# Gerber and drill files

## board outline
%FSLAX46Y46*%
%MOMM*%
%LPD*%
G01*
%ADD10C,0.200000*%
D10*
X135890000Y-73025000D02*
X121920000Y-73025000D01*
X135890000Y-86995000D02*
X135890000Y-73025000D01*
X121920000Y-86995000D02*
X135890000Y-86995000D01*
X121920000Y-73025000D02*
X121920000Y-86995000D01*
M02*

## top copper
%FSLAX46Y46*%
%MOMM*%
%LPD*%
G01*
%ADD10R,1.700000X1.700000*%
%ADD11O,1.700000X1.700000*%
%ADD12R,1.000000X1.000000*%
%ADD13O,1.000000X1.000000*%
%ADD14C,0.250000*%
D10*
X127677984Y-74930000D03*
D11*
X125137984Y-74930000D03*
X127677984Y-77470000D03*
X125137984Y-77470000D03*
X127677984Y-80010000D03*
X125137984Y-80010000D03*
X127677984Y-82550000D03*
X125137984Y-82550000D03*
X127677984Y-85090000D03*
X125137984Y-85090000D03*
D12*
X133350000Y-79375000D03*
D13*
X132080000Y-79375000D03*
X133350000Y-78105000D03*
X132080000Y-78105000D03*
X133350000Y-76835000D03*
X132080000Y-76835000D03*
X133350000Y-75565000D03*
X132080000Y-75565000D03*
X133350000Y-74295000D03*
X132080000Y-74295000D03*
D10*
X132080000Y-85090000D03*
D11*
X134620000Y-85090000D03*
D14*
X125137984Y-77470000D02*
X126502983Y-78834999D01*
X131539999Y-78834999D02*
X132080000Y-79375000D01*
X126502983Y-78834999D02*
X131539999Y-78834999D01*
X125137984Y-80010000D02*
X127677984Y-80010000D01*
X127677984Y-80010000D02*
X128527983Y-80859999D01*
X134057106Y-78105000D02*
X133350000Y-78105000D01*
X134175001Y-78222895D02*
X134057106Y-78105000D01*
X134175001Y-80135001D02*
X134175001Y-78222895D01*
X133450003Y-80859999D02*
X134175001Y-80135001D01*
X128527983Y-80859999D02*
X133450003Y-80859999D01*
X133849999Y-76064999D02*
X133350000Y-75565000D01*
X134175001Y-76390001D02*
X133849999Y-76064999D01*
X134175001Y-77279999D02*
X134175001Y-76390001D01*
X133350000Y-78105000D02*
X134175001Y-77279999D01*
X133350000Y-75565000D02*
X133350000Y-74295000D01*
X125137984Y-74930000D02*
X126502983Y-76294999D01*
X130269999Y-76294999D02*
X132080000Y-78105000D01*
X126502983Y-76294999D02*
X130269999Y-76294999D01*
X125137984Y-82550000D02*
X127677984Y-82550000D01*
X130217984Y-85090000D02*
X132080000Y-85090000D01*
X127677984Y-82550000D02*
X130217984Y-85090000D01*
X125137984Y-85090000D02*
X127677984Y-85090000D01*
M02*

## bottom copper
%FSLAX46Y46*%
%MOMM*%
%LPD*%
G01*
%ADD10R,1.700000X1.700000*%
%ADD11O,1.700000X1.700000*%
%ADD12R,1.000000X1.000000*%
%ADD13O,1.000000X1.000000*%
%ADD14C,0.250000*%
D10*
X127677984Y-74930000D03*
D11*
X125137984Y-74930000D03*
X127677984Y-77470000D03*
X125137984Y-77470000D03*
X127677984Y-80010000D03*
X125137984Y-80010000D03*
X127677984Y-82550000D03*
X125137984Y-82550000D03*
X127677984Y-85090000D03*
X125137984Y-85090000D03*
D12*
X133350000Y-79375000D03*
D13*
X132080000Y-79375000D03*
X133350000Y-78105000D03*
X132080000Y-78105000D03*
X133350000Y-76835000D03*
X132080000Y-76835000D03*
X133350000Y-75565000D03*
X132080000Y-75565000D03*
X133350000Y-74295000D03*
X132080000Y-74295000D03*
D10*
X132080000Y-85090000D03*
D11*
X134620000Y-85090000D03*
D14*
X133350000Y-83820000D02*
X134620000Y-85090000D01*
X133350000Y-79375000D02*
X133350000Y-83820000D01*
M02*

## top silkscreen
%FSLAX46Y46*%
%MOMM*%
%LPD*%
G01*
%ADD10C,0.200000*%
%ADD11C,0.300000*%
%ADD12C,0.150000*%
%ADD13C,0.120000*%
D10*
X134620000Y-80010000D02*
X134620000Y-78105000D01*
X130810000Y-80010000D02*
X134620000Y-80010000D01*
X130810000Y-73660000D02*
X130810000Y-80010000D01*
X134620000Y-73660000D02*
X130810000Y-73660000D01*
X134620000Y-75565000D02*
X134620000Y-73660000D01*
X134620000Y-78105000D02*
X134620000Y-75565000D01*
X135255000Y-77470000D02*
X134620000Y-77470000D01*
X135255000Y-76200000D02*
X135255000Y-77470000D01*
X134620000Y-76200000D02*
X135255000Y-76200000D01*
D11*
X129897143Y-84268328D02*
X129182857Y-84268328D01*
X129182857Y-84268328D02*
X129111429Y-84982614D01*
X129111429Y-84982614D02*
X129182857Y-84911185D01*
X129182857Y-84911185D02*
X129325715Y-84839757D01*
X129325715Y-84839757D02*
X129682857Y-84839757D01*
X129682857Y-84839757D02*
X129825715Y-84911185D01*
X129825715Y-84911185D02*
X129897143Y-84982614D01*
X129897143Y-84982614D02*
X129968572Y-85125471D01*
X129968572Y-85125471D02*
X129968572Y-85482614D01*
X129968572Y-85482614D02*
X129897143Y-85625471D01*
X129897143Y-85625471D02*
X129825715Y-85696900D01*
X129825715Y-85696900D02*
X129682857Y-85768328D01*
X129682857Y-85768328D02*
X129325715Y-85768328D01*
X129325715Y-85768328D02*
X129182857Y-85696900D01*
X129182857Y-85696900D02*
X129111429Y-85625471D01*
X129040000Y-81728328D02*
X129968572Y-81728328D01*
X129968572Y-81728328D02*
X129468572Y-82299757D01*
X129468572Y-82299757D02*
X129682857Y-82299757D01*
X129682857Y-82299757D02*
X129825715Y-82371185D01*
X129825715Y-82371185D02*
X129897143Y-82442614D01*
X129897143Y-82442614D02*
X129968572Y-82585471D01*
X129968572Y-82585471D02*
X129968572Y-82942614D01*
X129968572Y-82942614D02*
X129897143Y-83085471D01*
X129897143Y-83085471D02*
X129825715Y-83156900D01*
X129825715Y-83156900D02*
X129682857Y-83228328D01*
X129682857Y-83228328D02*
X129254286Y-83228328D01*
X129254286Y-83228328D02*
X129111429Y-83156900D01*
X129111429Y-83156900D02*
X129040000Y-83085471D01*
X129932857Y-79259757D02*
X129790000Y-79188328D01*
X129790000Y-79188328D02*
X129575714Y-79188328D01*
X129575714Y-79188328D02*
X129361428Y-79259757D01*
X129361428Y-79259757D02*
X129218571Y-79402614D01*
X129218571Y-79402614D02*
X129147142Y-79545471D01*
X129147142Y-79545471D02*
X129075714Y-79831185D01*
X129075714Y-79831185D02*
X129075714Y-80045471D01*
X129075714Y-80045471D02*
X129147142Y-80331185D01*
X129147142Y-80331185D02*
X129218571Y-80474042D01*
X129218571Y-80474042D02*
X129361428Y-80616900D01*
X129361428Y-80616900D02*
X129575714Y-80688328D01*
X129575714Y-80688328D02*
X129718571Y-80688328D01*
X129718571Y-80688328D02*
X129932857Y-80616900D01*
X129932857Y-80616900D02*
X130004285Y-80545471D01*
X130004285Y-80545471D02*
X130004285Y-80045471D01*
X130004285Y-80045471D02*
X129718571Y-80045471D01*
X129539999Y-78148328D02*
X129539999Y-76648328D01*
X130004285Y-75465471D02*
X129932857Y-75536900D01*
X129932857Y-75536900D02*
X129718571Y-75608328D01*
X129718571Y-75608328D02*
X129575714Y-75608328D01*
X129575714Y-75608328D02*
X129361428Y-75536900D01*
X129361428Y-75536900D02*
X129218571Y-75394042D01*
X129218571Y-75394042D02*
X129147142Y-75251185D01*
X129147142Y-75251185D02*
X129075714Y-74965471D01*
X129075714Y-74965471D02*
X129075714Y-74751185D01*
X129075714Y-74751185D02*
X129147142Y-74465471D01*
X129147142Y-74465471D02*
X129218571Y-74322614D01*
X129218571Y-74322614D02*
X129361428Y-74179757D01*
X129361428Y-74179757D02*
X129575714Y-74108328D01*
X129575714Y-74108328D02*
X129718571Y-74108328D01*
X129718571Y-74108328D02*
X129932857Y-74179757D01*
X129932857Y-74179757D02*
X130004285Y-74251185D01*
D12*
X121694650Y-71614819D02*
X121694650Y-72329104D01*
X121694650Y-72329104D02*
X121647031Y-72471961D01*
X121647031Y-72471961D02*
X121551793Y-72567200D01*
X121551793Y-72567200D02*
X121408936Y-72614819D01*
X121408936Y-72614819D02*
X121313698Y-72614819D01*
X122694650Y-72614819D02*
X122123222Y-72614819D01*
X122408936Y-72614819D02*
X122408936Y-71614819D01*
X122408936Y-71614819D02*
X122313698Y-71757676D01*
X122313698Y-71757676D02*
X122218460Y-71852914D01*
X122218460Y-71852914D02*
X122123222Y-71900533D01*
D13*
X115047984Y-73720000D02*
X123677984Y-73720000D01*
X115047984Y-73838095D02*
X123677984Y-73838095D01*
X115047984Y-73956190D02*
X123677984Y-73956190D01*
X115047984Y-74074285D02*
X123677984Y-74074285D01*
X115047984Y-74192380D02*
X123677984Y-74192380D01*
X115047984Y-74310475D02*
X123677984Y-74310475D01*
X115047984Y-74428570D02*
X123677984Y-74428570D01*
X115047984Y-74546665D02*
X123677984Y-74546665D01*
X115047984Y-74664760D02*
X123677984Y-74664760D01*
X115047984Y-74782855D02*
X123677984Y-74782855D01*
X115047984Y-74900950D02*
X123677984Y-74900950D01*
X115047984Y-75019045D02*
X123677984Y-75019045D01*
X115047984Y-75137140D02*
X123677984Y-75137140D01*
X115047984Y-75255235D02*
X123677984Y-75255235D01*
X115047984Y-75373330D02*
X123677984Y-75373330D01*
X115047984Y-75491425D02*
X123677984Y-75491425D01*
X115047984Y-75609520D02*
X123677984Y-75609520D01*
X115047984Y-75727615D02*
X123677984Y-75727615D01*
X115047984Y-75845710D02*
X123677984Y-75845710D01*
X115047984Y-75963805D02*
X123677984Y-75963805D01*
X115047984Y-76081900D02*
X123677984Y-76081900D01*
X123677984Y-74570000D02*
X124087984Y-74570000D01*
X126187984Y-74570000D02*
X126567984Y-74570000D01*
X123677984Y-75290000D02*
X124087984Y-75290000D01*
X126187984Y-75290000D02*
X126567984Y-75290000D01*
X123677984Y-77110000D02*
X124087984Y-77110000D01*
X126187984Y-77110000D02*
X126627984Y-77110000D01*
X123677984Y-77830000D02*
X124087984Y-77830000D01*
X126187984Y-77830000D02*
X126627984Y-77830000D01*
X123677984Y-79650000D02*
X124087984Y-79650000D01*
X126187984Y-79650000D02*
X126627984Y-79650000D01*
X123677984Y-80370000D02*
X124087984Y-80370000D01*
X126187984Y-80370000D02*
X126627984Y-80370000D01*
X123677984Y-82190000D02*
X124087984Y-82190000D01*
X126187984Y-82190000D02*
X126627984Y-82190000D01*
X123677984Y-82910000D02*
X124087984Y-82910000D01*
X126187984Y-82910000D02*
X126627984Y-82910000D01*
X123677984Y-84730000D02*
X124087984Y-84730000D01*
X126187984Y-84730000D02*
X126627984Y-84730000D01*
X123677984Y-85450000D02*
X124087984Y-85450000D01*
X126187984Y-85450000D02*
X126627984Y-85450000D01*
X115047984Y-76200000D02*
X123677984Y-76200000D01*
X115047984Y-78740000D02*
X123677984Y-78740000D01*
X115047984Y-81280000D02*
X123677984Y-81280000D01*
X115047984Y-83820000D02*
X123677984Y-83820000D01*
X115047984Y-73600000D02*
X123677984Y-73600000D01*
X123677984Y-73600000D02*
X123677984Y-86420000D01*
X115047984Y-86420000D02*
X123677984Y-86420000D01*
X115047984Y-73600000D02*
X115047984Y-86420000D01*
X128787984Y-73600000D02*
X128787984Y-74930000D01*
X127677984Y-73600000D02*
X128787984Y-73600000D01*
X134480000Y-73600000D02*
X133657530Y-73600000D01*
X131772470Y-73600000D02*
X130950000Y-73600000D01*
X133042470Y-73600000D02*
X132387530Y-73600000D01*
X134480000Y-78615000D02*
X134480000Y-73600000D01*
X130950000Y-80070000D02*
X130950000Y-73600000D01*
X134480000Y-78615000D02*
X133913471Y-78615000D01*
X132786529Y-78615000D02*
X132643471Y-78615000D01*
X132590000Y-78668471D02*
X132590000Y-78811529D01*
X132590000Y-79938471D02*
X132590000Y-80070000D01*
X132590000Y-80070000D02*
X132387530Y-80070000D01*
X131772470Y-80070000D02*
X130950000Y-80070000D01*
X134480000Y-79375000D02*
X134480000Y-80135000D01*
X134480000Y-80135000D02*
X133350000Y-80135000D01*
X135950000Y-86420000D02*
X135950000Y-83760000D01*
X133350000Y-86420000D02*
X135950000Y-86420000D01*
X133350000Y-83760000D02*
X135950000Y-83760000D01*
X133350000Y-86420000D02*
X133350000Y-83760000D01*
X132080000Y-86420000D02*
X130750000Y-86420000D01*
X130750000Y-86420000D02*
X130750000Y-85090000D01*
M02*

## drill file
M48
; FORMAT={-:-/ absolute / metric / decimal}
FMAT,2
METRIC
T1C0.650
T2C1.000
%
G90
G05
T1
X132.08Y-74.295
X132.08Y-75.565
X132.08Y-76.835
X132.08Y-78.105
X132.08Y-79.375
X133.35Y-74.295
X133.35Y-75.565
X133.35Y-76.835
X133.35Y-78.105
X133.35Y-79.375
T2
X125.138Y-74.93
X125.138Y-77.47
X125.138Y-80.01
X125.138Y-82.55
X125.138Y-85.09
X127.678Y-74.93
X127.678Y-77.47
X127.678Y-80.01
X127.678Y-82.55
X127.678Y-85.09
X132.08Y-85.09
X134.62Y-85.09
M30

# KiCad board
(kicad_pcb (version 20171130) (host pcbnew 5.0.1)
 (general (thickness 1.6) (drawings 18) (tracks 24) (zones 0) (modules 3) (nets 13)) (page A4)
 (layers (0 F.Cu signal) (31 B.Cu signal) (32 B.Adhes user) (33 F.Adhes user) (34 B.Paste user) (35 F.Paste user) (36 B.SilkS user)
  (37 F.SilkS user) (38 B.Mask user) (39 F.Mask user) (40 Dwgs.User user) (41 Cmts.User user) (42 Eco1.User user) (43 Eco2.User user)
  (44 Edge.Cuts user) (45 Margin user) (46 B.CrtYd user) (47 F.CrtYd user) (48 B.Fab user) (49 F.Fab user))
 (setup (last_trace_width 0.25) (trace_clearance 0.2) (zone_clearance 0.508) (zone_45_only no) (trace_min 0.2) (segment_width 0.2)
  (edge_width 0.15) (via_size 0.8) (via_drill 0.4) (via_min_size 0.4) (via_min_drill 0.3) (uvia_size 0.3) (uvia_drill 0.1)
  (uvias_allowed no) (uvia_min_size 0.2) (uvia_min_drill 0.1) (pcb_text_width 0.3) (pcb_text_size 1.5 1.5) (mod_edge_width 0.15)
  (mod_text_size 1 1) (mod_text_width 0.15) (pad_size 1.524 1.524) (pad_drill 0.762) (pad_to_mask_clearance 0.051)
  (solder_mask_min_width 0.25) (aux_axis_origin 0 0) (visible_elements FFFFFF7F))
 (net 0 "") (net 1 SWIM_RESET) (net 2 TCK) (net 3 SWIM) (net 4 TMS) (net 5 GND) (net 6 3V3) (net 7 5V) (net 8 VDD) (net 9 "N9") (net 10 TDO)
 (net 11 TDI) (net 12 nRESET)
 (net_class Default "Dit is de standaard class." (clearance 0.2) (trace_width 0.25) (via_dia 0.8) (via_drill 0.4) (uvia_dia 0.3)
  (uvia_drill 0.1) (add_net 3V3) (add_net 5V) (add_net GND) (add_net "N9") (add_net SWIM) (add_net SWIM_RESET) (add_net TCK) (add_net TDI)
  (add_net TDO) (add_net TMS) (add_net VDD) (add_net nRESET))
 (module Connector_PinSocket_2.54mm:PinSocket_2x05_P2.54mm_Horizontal (layer F.Cu) (at 127.677984 74.93)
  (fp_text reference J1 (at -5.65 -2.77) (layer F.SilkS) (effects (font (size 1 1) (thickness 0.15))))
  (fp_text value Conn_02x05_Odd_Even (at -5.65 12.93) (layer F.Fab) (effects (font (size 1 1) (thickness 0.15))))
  (fp_line (start -12.63 -1.21) (end -4 -1.21) (layer F.SilkS) (width 0.12))
  (fp_line (start -12.63 -1.091905) (end -4 -1.091905) (layer F.SilkS) (width 0.12))
  (fp_line (start -12.63 -0.97381) (end -4 -0.97381) (layer F.SilkS) (width 0.12))
  (fp_line (start -12.63 -0.855715) (end -4 -0.855715) (layer F.SilkS) (width 0.12))
  (fp_line (start -12.63 -0.73762) (end -4 -0.73762) (layer F.SilkS) (width 0.12))
  (fp_line (start -12.63 -0.619525) (end -4 -0.619525) (layer F.SilkS) (width 0.12))
  (fp_line (start -12.63 -0.50143) (end -4 -0.50143) (layer F.SilkS) (width 0.12))
  (fp_line (start -12.63 -0.383335) (end -4 -0.383335) (layer F.SilkS) (width 0.12))
  (fp_line (start -12.63 -0.26524) (end -4 -0.26524) (layer F.SilkS) (width 0.12))
  (fp_line (start -12.63 -0.147145) (end -4 -0.147145) (layer F.SilkS) (width 0.12))
  (fp_line (start -12.63 -0.02905) (end -4 -0.02905) (layer F.SilkS) (width 0.12))
  (fp_line (start -12.63 0.089045) (end -4 0.089045) (layer F.SilkS) (width 0.12))
  (fp_line (start -12.63 0.20714) (end -4 0.20714) (layer F.SilkS) (width 0.12))
  (fp_line (start -12.63 0.325235) (end -4 0.325235) (layer F.SilkS) (width 0.12))
  (fp_line (start -12.63 0.44333) (end -4 0.44333) (layer F.SilkS) (width 0.12))
  (fp_line (start -12.63 0.561425) (end -4 0.561425) (layer F.SilkS) (width 0.12))
  (fp_line (start -12.63 0.67952) (end -4 0.67952) (layer F.SilkS) (width 0.12))
  (fp_line (start -12.63 0.797615) (end -4 0.797615) (layer F.SilkS) (width 0.12))
  (fp_line (start -12.63 0.91571) (end -4 0.91571) (layer F.SilkS) (width 0.12))
  (fp_line (start -12.63 1.033805) (end -4 1.033805) (layer F.SilkS) (width 0.12))
  (fp_line (start -12.63 1.1519) (end -4 1.1519) (layer F.SilkS) (width 0.12))
  (fp_line (start -4 -0.36) (end -3.59 -0.36) (layer F.SilkS) (width 0.12))
  (fp_line (start -1.49 -0.36) (end -1.11 -0.36) (layer F.SilkS) (width 0.12))
  (fp_line (start -4 0.36) (end -3.59 0.36) (layer F.SilkS) (width 0.12))
  (fp_line (start -1.49 0.36) (end -1.11 0.36) (layer F.SilkS) (width 0.12))
  (fp_line (start -4 2.18) (end -3.59 2.18) (layer F.SilkS) (width 0.12))
  (fp_line (start -1.49 2.18) (end -1.05 2.18) (layer F.SilkS) (width 0.12))
  (fp_line (start -4 2.9) (end -3.59 2.9) (layer F.SilkS) (width 0.12))
  (fp_line (start -1.49 2.9) (end -1.05 2.9) (layer F.SilkS) (width 0.12))
  (fp_line (start -4 4.72) (end -3.59 4.72) (layer F.SilkS) (width 0.12))
  (fp_line (start -1.49 4.72) (end -1.05 4.72) (layer F.SilkS) (width 0.12))
  (fp_line (start -4 5.44) (end -3.59 5.44) (layer F.SilkS) (width 0.12))
  (fp_line (start -1.49 5.44) (end -1.05 5.44) (layer F.SilkS) (width 0.12))
  (fp_line (start -4 7.26) (end -3.59 7.26) (layer F.SilkS) (width 0.12))
  (fp_line (start -1.49 7.26) (end -1.05 7.26) (layer F.SilkS) (width 0.12))
  (fp_line (start -4 7.98) (end -3.59 7.98) (layer F.SilkS) (width 0.12))
  (fp_line (start -1.49 7.98) (end -1.05 7.98) (layer F.SilkS) (width 0.12))
  (fp_line (start -4 9.8) (end -3.59 9.8) (layer F.SilkS) (width 0.12))
  (fp_line (start -1.49 9.8) (end -1.05 9.8) (layer F.SilkS) (width 0.12))
  (fp_line (start -4 10.52) (end -3.59 10.52) (layer F.SilkS) (width 0.12))
  (fp_line (start -1.49 10.52) (end -1.05 10.52) (layer F.SilkS) (width 0.12))
  (fp_line (start -12.63 1.27) (end -4 1.27) (layer F.SilkS) (width 0.12))
  (fp_line (start -12.63 3.81) (end -4 3.81) (layer F.SilkS) (width 0.12))
  (fp_line (start -12.63 6.35) (end -4 6.35) (layer F.SilkS) (width 0.12))
  (fp_line (start -12.63 8.89) (end -4 8.89) (layer F.SilkS) (width 0.12))
  (fp_line (start -12.63 -1.33) (end -4 -1.33) (layer F.SilkS) (width 0.12))
  (fp_line (start -4 -1.33) (end -4 11.49) (layer F.SilkS) (width 0.12))
  (fp_line (start -12.63 11.49) (end -4 11.49) (layer F.SilkS) (width 0.12))
  (fp_line (start -12.63 -1.33) (end -12.63 11.49) (layer F.SilkS) (width 0.12))
  (fp_line (start 1.11 -1.33) (end 1.11 0) (layer F.SilkS) (width 0.12))
  (fp_line (start 0 -1.33) (end 1.11 -1.33) (layer F.SilkS) (width 0.12))
  (pad 1 thru_hole rect (at 0 0) (size 1.7 1.7) (drill 1) (layers *.Cu *.Mask) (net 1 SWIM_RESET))
  (pad 2 thru_hole oval (at -2.54 0) (size 1.7 1.7) (drill 1) (layers *.Cu *.Mask) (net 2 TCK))
  (pad 3 thru_hole oval (at 0 2.54) (size 1.7 1.7) (drill 1) (layers *.Cu *.Mask) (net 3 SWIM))
  (pad 4 thru_hole oval (at -2.54 2.54) (size 1.7 1.7) (drill 1) (layers *.Cu *.Mask) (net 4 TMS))
  (pad 5 thru_hole oval (at 0 5.08) (size 1.7 1.7) (drill 1) (layers *.Cu *.Mask) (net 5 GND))
  (pad 6 thru_hole oval (at -2.54 5.08) (size 1.7 1.7) (drill 1) (layers *.Cu *.Mask) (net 5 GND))
  (pad 7 thru_hole oval (at 0 7.62) (size 1.7 1.7) (drill 1) (layers *.Cu *.Mask) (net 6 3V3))
  (pad 8 thru_hole oval (at -2.54 7.62) (size 1.7 1.7) (drill 1) (layers *.Cu *.Mask) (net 6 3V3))
  (pad 9 thru_hole oval (at 0 10.16) (size 1.7 1.7) (drill 1) (layers *.Cu *.Mask) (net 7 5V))
  (pad 10 thru_hole oval (at -2.54 10.16) (size 1.7 1.7) (drill 1) (layers *.Cu *.Mask) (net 7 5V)))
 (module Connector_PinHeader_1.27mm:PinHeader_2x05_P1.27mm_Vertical (layer F.Cu) (at 133.35 79.375 180)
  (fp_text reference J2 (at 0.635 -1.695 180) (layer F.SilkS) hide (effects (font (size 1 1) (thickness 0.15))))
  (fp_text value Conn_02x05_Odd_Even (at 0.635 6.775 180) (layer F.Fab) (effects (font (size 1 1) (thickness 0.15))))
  (fp_line (start -1.13 5.775) (end -0.30753 5.775) (layer F.SilkS) (width 0.12))
  (fp_line (start 1.57753 5.775) (end 2.4 5.775) (layer F.SilkS) (width 0.12))
  (fp_line (start 0.30753 5.775) (end 0.96247 5.775) (layer F.SilkS) (width 0.12))
  (fp_line (start -1.13 0.76) (end -1.13 5.775) (layer F.SilkS) (width 0.12))
  (fp_line (start 2.4 -0.695) (end 2.4 5.775) (layer F.SilkS) (width 0.12))
  (fp_line (start -1.13 0.76) (end -0.563471 0.76) (layer F.SilkS) (width 0.12))
  (fp_line (start 0.563471 0.76) (end 0.706529 0.76) (layer F.SilkS) (width 0.12))
  (fp_line (start 0.76 0.706529) (end 0.76 0.563471) (layer F.SilkS) (width 0.12))
  (fp_line (start 0.76 -0.563471) (end 0.76 -0.695) (layer F.SilkS) (width 0.12))
  (fp_line (start 0.76 -0.695) (end 0.96247 -0.695) (layer F.SilkS) (width 0.12))
  (fp_line (start 1.57753 -0.695) (end 2.4 -0.695) (layer F.SilkS) (width 0.12))
  (fp_line (start -1.13 0) (end -1.13 -0.76) (layer F.SilkS) (width 0.12))
  (fp_line (start -1.13 -0.76) (end 0 -0.76) (layer F.SilkS) (width 0.12))
  (pad 1 thru_hole rect (at 0 0 180) (size 1 1) (drill 0.65) (layers *.Cu *.Mask) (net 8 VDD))
  (pad 2 thru_hole oval (at 1.27 0 180) (size 1 1) (drill 0.65) (layers *.Cu *.Mask) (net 4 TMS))
  (pad 3 thru_hole oval (at 0 1.27 180) (size 1 1) (drill 0.65) (layers *.Cu *.Mask) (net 5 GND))
  (pad 4 thru_hole oval (at 1.27 1.27 180) (size 1 1) (drill 0.65) (layers *.Cu *.Mask) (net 2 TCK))
  (pad 5 thru_hole oval (at 0 2.54 180) (size 1 1) (drill 0.65) (layers *.Cu *.Mask) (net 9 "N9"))
  (pad 6 thru_hole oval (at 1.27 2.54 180) (size 1 1) (drill 0.65) (layers *.Cu *.Mask) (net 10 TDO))
  (pad 7 thru_hole oval (at 0 3.81 180) (size 1 1) (drill 0.65) (layers *.Cu *.Mask) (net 5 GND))
  (pad 8 thru_hole oval (at 1.27 3.81 180) (size 1 1) (drill 0.65) (layers *.Cu *.Mask) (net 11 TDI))
  (pad 9 thru_hole oval (at 0 5.08 180) (size 1 1) (drill 0.65) (layers *.Cu *.Mask) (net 5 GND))
  (pad 10 thru_hole oval (at 1.27 5.08 180) (size 1 1) (drill 0.65) (layers *.Cu *.Mask) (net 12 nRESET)))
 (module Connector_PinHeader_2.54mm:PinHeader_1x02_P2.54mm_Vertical (layer F.Cu) (at 132.08 85.09 90)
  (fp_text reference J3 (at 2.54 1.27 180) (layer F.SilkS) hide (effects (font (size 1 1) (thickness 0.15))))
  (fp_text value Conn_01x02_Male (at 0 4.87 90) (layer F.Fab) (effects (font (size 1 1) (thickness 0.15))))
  (fp_line (start -1.33 3.87) (end 1.33 3.87) (layer F.SilkS) (width 0.12))
  (fp_line (start -1.33 1.27) (end -1.33 3.87) (layer F.SilkS) (width 0.12))
  (fp_line (start 1.33 1.27) (end 1.33 3.87) (layer F.SilkS) (width 0.12))
  (fp_line (start -1.33 1.27) (end 1.33 1.27) (layer F.SilkS) (width 0.12))
  (fp_line (start -1.33 0) (end -1.33 -1.33) (layer F.SilkS) (width 0.12))
  (fp_line (start -1.33 -1.33) (end 0 -1.33) (layer F.SilkS) (width 0.12))
  (pad 1 thru_hole rect (at 0 0 90) (size 1.7 1.7) (drill 1) (layers *.Cu *.Mask) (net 6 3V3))
  (pad 2 thru_hole oval (at 0 2.54 90) (size 1.7 1.7) (drill 1) (layers *.Cu *.Mask) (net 8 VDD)))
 (gr_line (start 134.62 80.01) (end 134.62 78.105) (layer F.SilkS) (width 0.2))
 (gr_line (start 130.81 80.01) (end 134.62 80.01) (layer F.SilkS) (width 0.2))
 (gr_line (start 130.81 73.66) (end 130.81 80.01) (layer F.SilkS) (width 0.2))
 (gr_line (start 134.62 73.66) (end 130.81 73.66) (layer F.SilkS) (width 0.2))
 (gr_line (start 134.62 75.565) (end 134.62 73.66) (layer F.SilkS) (width 0.2))
 (gr_line (start 134.62 78.105) (end 134.62 75.565) (layer F.SilkS) (width 0.2))
 (gr_line (start 135.255 77.47) (end 134.62 77.47) (layer F.SilkS) (width 0.2))
 (gr_line (start 135.255 76.2) (end 135.255 77.47) (layer F.SilkS) (width 0.2))
 (gr_line (start 134.62 76.2) (end 135.255 76.2) (layer F.SilkS) (width 0.2))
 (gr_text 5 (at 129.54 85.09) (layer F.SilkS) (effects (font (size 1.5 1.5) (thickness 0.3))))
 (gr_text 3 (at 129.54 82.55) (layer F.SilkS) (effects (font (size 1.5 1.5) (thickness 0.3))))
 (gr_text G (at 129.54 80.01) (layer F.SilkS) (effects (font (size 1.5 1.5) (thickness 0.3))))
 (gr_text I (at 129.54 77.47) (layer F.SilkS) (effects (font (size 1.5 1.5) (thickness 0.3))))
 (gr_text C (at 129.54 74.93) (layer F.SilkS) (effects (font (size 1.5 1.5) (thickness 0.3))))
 (gr_line (start 135.89 73.025) (end 121.92 73.025) (layer Edge.Cuts) (width 0.2))
 (gr_line (start 135.89 86.995) (end 135.89 73.025) (layer Edge.Cuts) (width 0.2))
 (gr_line (start 121.92 86.995) (end 135.89 86.995) (layer Edge.Cuts) (width 0.2))
 (gr_line (start 121.92 73.025) (end 121.92 86.995) (layer Edge.Cuts) (width 0.2))
 (segment (start 125.137984 77.47) (end 126.502983 78.834999) (width 0.25) (layer F.Cu) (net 4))
 (segment (start 131.539999 78.834999) (end 132.08 79.375) (width 0.25) (layer F.Cu) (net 4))
 (segment (start 126.502983 78.834999) (end 131.539999 78.834999) (width 0.25) (layer F.Cu) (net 4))
 (segment (start 125.137984 80.01) (end 127.677984 80.01) (width 0.25) (layer F.Cu) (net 5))
 (segment (start 127.677984 80.01) (end 128.527983 80.859999) (width 0.25) (layer F.Cu) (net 5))
 (segment (start 134.057106 78.105) (end 133.35 78.105) (width 0.25) (layer F.Cu) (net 5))
 (segment (start 134.175001 78.222895) (end 134.057106 78.105) (width 0.25) (layer F.Cu) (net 5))
 (segment (start 134.175001 80.135001) (end 134.175001 78.222895) (width 0.25) (layer F.Cu) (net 5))
 (segment (start 133.450003 80.859999) (end 134.175001 80.135001) (width 0.25) (layer F.Cu) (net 5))
 (segment (start 128.527983 80.859999) (end 133.450003 80.859999) (width 0.25) (layer F.Cu) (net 5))
 (segment (start 133.849999 76.064999) (end 133.35 75.565) (width 0.25) (layer F.Cu) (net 5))
 (segment (start 134.175001 76.390001) (end 133.849999 76.064999) (width 0.25) (layer F.Cu) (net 5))
 (segment (start 134.175001 77.279999) (end 134.175001 76.390001) (width 0.25) (layer F.Cu) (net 5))
 (segment (start 133.35 78.105) (end 134.175001 77.279999) (width 0.25) (layer F.Cu) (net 5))
 (segment (start 133.35 75.565) (end 133.35 74.295) (width 0.25) (layer F.Cu) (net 5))
 (segment (start 125.137984 74.93) (end 126.502983 76.294999) (width 0.25) (layer F.Cu) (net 2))
 (segment (start 130.269999 76.294999) (end 132.08 78.105) (width 0.25) (layer F.Cu) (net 2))
 (segment (start 126.502983 76.294999) (end 130.269999 76.294999) (width 0.25) (layer F.Cu) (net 2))
 (segment (start 125.137984 82.55) (end 127.677984 82.55) (width 0.25) (layer F.Cu) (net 6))
 (segment (start 130.217984 85.09) (end 132.08 85.09) (width 0.25) (layer F.Cu) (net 6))
 (segment (start 127.677984 82.55) (end 130.217984 85.09) (width 0.25) (layer F.Cu) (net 6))
 (segment (start 125.137984 85.09) (end 127.677984 85.09) (width 0.25) (layer F.Cu) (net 7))
 (segment (start 133.35 83.82) (end 134.62 85.09) (width 0.25) (layer B.Cu) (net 8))
 (segment (start 133.35 79.375) (end 133.35 83.82) (width 0.25) (layer B.Cu) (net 8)))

